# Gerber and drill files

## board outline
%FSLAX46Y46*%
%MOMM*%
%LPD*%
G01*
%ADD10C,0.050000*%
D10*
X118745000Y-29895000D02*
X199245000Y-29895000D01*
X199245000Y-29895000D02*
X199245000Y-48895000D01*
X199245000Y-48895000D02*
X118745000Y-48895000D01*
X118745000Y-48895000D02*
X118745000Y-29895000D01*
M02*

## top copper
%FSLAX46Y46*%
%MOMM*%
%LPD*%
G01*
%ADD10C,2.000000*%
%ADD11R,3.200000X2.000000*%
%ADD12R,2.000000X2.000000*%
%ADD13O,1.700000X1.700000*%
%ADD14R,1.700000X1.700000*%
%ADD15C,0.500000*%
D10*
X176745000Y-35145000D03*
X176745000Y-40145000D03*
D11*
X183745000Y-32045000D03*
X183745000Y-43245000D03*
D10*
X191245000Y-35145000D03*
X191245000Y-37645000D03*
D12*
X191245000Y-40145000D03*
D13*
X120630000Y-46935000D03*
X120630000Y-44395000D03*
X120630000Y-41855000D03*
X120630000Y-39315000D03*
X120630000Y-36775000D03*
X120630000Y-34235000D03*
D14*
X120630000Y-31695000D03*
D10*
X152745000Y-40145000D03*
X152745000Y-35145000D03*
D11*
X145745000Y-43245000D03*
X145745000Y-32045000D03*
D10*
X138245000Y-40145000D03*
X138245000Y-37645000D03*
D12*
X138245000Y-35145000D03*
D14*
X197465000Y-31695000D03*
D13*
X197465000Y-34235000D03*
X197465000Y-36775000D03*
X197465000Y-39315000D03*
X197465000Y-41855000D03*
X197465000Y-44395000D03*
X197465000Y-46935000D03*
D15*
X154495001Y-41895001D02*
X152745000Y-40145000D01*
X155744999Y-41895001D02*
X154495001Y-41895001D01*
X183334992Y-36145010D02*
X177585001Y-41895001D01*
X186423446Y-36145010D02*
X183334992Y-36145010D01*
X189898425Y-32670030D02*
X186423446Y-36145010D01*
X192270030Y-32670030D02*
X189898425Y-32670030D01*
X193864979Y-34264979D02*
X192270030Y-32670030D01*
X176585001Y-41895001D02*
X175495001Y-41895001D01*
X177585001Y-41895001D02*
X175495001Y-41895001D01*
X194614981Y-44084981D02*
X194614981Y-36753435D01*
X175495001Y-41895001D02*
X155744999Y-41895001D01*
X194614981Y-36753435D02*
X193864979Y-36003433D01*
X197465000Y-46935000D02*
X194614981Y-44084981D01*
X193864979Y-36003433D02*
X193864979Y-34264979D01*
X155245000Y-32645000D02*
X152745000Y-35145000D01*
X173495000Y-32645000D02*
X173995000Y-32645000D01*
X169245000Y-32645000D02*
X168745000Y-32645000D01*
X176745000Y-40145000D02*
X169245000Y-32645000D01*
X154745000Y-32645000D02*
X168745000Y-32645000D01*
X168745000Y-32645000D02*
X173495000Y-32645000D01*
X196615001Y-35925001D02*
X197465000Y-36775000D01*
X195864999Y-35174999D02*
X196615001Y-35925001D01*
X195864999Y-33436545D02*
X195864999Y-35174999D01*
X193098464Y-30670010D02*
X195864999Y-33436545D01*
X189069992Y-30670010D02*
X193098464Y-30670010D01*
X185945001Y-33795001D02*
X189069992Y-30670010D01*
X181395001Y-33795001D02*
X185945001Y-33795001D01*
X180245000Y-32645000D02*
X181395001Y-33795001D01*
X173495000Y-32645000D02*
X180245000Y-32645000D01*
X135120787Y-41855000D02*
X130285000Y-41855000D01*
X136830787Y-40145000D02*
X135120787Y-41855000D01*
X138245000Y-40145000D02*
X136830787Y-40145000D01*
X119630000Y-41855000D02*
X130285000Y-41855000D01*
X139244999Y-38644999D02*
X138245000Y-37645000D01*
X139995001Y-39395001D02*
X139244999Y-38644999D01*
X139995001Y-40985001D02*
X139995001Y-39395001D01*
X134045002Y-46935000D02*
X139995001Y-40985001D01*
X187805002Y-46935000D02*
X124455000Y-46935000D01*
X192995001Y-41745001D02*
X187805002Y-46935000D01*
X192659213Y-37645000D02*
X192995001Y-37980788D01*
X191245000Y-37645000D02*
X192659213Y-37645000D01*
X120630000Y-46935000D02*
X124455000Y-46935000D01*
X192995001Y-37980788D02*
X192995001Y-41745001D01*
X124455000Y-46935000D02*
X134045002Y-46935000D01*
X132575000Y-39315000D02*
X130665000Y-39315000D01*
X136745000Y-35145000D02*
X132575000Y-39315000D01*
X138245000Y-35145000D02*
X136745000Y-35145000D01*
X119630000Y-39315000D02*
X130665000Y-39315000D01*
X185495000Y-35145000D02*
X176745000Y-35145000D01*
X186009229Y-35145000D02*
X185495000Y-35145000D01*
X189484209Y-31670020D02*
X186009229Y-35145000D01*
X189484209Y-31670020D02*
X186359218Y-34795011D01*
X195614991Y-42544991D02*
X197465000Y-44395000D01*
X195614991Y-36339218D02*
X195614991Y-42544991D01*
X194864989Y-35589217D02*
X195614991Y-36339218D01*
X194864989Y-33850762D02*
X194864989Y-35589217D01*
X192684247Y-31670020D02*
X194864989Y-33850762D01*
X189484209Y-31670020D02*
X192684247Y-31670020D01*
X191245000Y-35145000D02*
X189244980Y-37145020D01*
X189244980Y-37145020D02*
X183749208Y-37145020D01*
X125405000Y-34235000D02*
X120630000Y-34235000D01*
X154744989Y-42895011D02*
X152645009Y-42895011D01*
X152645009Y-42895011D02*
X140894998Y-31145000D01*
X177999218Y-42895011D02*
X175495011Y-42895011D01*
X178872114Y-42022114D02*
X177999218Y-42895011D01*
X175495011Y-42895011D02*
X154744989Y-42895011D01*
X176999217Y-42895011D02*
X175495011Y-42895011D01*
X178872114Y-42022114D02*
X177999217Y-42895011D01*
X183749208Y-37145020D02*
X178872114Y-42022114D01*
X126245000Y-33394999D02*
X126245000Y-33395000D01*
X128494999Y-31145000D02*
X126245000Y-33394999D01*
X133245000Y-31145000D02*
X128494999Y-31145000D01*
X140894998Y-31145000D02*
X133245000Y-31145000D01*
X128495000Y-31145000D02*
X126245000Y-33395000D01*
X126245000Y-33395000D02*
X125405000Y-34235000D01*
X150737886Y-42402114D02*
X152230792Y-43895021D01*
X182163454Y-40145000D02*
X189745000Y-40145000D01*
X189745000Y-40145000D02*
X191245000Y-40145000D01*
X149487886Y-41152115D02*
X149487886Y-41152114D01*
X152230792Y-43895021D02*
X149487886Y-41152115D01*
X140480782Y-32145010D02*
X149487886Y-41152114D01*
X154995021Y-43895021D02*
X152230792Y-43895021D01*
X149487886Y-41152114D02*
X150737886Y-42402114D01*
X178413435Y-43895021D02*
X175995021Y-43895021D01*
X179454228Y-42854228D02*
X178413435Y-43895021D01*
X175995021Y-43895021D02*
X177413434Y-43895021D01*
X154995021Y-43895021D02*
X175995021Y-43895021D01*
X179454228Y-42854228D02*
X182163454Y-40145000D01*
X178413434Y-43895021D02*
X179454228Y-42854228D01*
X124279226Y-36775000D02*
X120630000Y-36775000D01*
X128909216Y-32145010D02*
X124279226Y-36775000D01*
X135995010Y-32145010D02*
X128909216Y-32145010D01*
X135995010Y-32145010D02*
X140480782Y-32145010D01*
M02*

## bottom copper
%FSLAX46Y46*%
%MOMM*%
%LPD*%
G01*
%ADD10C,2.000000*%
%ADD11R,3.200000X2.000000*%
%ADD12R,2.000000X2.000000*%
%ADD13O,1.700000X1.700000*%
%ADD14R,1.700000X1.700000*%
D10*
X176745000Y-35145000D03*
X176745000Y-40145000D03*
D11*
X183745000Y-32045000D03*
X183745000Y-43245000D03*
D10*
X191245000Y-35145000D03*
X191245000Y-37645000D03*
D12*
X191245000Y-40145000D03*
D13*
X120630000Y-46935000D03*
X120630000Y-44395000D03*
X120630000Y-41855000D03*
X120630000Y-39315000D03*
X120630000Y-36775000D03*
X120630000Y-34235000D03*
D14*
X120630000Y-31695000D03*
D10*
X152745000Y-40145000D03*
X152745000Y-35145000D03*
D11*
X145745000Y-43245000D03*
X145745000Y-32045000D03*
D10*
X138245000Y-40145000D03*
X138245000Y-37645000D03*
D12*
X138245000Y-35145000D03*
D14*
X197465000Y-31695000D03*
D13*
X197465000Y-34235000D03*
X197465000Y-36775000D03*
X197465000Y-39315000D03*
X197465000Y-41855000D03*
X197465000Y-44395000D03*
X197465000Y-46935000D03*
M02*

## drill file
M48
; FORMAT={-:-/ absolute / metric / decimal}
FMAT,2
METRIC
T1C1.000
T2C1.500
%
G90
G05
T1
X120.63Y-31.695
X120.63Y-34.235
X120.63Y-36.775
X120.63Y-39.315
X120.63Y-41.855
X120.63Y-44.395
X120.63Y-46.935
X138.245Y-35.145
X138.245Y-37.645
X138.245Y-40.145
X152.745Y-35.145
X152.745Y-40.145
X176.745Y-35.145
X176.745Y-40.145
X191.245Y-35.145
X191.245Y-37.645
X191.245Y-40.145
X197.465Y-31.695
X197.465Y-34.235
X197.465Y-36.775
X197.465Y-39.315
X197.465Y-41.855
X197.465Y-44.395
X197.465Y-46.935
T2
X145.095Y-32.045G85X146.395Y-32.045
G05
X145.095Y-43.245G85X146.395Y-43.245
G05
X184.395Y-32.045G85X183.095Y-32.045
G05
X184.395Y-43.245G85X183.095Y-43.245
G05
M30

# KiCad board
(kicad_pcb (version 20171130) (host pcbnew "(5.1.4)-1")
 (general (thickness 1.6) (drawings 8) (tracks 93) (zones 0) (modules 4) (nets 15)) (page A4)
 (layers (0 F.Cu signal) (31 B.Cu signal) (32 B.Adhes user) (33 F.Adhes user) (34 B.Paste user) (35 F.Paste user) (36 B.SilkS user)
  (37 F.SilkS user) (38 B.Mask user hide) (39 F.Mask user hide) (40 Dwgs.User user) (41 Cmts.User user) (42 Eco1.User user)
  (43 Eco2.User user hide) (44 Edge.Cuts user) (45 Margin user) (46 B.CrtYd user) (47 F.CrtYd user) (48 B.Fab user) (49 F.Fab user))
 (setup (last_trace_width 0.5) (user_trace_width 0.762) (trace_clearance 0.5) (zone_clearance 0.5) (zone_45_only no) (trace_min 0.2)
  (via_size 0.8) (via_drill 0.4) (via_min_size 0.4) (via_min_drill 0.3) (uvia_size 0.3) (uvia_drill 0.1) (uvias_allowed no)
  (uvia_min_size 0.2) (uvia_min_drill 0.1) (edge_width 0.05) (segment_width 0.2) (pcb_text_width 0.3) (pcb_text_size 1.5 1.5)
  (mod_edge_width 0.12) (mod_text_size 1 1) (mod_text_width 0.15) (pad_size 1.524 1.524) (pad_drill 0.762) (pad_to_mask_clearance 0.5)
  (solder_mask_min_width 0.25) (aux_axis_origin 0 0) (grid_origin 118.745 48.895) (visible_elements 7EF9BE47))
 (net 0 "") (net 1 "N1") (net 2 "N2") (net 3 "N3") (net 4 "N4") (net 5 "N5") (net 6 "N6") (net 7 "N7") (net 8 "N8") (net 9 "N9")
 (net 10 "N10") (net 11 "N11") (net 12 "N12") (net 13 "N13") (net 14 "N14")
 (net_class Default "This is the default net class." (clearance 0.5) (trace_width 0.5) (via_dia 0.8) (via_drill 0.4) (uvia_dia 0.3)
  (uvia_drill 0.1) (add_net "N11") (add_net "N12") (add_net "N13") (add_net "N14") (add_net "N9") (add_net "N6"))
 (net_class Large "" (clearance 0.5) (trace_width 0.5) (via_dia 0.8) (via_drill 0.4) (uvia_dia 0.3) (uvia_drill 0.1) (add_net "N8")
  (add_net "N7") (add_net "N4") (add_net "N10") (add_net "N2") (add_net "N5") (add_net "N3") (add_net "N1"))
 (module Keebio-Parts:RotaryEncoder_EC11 (layer F.Cu) (at 183.745 37.645 180)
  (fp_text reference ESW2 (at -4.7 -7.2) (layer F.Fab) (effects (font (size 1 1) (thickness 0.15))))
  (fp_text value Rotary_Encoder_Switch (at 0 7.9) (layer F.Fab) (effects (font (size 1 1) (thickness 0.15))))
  (pad S1 thru_hole circle (at 7 2.5 180) (size 2 2) (drill 1) (layers *.Cu *.Mask) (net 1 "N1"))
  (pad S2 thru_hole circle (at 7 -2.5 180) (size 2 2) (drill 1) (layers *.Cu *.Mask) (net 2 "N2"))
  (pad MP thru_hole rect (at 0 5.6 180) (size 3.2 2) (drill oval 2.8 1.5) (layers *.Cu *.Mask))
  (pad MP thru_hole rect (at 0 -5.6 180) (size 3.2 2) (drill oval 2.8 1.5) (layers *.Cu *.Mask))
  (pad B thru_hole circle (at -7.5 2.5 180) (size 2 2) (drill 1) (layers *.Cu *.Mask) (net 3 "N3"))
  (pad C thru_hole circle (at -7.5 0 180) (size 2 2) (drill 1) (layers *.Cu *.Mask) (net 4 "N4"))
  (pad A thru_hole rect (at -7.5 -2.5 180) (size 2 2) (drill 1) (layers *.Cu *.Mask) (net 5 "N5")))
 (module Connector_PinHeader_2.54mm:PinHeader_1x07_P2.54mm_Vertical (layer F.Cu) (at 120.63 31.695)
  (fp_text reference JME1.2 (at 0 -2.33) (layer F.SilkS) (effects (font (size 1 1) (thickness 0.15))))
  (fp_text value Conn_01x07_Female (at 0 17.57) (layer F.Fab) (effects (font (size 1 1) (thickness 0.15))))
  (pad 7 thru_hole oval (at 0 15.24) (size 1.7 1.7) (drill 1) (layers *.Cu *.Mask) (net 4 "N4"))
  (pad 6 thru_hole oval (at 0 12.7) (size 1.7 1.7) (drill 1) (layers *.Cu *.Mask) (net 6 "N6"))
  (pad 5 thru_hole oval (at 0 10.16) (size 1.7 1.7) (drill 1) (layers *.Cu *.Mask) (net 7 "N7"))
  (pad 4 thru_hole oval (at 0 7.62) (size 1.7 1.7) (drill 1) (layers *.Cu *.Mask) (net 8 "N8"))
  (pad 3 thru_hole oval (at 0 5.08) (size 1.7 1.7) (drill 1) (layers *.Cu *.Mask) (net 5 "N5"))
  (pad 2 thru_hole oval (at 0 2.54) (size 1.7 1.7) (drill 1) (layers *.Cu *.Mask) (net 3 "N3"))
  (pad 1 thru_hole rect (at 0 0) (size 1.7 1.7) (drill 1) (layers *.Cu *.Mask) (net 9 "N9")))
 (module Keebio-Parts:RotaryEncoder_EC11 (layer F.Cu) (at 145.745 37.645)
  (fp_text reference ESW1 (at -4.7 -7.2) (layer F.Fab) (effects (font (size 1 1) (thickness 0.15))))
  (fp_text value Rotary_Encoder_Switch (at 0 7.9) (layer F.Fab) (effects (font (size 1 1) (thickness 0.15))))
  (pad S1 thru_hole circle (at 7 2.5) (size 2 2) (drill 1) (layers *.Cu *.Mask) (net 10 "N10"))
  (pad S2 thru_hole circle (at 7 -2.5) (size 2 2) (drill 1) (layers *.Cu *.Mask) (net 2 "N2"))
  (pad MP thru_hole rect (at 0 5.6) (size 3.2 2) (drill oval 2.8 1.5) (layers *.Cu *.Mask))
  (pad MP thru_hole rect (at 0 -5.6) (size 3.2 2) (drill oval 2.8 1.5) (layers *.Cu *.Mask))
  (pad B thru_hole circle (at -7.5 2.5) (size 2 2) (drill 1) (layers *.Cu *.Mask) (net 7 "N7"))
  (pad C thru_hole circle (at -7.5 0) (size 2 2) (drill 1) (layers *.Cu *.Mask) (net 4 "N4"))
  (pad A thru_hole rect (at -7.5 -2.5) (size 2 2) (drill 1) (layers *.Cu *.Mask) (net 8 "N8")))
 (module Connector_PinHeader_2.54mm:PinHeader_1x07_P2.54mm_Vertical (layer F.Cu) (at 197.465 31.695)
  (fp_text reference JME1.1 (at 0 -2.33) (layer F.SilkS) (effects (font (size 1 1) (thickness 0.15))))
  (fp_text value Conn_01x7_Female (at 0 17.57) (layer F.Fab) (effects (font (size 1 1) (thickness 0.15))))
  (pad 1 thru_hole rect (at 0 0) (size 1.7 1.7) (drill 1) (layers *.Cu *.Mask) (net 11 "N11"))
  (pad 2 thru_hole oval (at 0 2.54) (size 1.7 1.7) (drill 1) (layers *.Cu *.Mask) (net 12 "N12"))
  (pad 3 thru_hole oval (at 0 5.08) (size 1.7 1.7) (drill 1) (layers *.Cu *.Mask) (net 2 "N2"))
  (pad 4 thru_hole oval (at 0 7.62) (size 1.7 1.7) (drill 1) (layers *.Cu *.Mask) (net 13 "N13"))
  (pad 5 thru_hole oval (at 0 10.16) (size 1.7 1.7) (drill 1) (layers *.Cu *.Mask) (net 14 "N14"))
  (pad 6 thru_hole oval (at 0 12.7) (size 1.7 1.7) (drill 1) (layers *.Cu *.Mask) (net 1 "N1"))
  (pad 7 thru_hole oval (at 0 15.24) (size 1.7 1.7) (drill 1) (layers *.Cu *.Mask) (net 10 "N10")))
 (gr_line (start 118.745 29.895) (end 199.245 29.895) (layer Edge.Cuts) (width 0.05))
 (gr_line (start 199.245 29.895) (end 199.245 48.895) (layer Edge.Cuts) (width 0.05))
 (gr_line (start 199.245 48.895) (end 118.745 48.895) (layer Edge.Cuts) (width 0.05))
 (gr_line (start 118.745 48.895) (end 118.745 29.895) (layer Edge.Cuts) (width 0.05))
 (segment (start 154.495001 41.895001) (end 152.745 40.145) (width 0.5) (layer F.Cu) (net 10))
 (segment (start 155.744999 41.895001) (end 154.495001 41.895001) (width 0.5) (layer F.Cu) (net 10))
 (segment (start 183.334992 36.14501) (end 177.585001 41.895001) (width 0.5) (layer F.Cu) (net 10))
 (segment (start 186.423446 36.14501) (end 183.334992 36.14501) (width 0.5) (layer F.Cu) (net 10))
 (segment (start 189.898425 32.67003) (end 186.423446 36.14501) (width 0.5) (layer F.Cu) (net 10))
 (segment (start 192.27003 32.67003) (end 189.898425 32.67003) (width 0.5) (layer F.Cu) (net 10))
 (segment (start 193.864979 34.264979) (end 192.27003 32.67003) (width 0.5) (layer F.Cu) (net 10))
 (segment (start 176.585001 41.895001) (end 175.495001 41.895001) (width 0.5) (layer F.Cu) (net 10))
 (segment (start 177.585001 41.895001) (end 175.495001 41.895001) (width 0.5) (layer F.Cu) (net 10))
 (segment (start 194.614981 44.084981) (end 194.614981 36.753435) (width 0.5) (layer F.Cu) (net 10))
 (segment (start 175.495001 41.895001) (end 155.744999 41.895001) (width 0.5) (layer F.Cu) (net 10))
 (segment (start 194.614981 36.753435) (end 193.864979 36.003433) (width 0.5) (layer F.Cu) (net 10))
 (segment (start 197.465 46.935) (end 194.614981 44.084981) (width 0.5) (layer F.Cu) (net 10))
 (segment (start 193.864979 36.003433) (end 193.864979 34.264979) (width 0.5) (layer F.Cu) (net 10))
 (segment (start 155.245 32.645) (end 152.745 35.145) (width 0.5) (layer F.Cu) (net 2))
 (segment (start 173.495 32.645) (end 173.995 32.645) (width 0.5) (layer F.Cu) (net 2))
 (segment (start 169.245 32.645) (end 168.745 32.645) (width 0.5) (layer F.Cu) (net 2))
 (segment (start 176.745 40.145) (end 169.245 32.645) (width 0.5) (layer F.Cu) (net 2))
 (segment (start 154.745 32.645) (end 168.745 32.645) (width 0.5) (layer F.Cu) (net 2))
 (segment (start 168.745 32.645) (end 173.495 32.645) (width 0.5) (layer F.Cu) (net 2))
 (segment (start 196.615001 35.925001) (end 197.465 36.775) (width 0.5) (layer F.Cu) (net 2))
 (segment (start 195.864999 35.174999) (end 196.615001 35.925001) (width 0.5) (layer F.Cu) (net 2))
 (segment (start 195.864999 33.436545) (end 195.864999 35.174999) (width 0.5) (layer F.Cu) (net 2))
 (segment (start 193.098464 30.67001) (end 195.864999 33.436545) (width 0.5) (layer F.Cu) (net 2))
 (segment (start 189.069992 30.67001) (end 193.098464 30.67001) (width 0.5) (layer F.Cu) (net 2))
 (segment (start 185.945001 33.795001) (end 189.069992 30.67001) (width 0.5) (layer F.Cu) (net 2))
 (segment (start 181.395001 33.795001) (end 185.945001 33.795001) (width 0.5) (layer F.Cu) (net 2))
 (segment (start 180.245 32.645) (end 181.395001 33.795001) (width 0.5) (layer F.Cu) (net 2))
 (segment (start 173.495 32.645) (end 180.245 32.645) (width 0.5) (layer F.Cu) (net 2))
 (segment (start 135.120787 41.855) (end 130.285 41.855) (width 0.5) (layer F.Cu) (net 7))
 (segment (start 136.830787 40.145) (end 135.120787 41.855) (width 0.5) (layer F.Cu) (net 7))
 (segment (start 138.245 40.145) (end 136.830787 40.145) (width 0.5) (layer F.Cu) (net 7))
 (segment (start 119.63 41.855) (end 130.285 41.855) (width 0.5) (layer F.Cu) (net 7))
 (segment (start 139.244999 38.644999) (end 138.245 37.645) (width 0.5) (layer F.Cu) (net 4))
 (segment (start 139.995001 39.395001) (end 139.244999 38.644999) (width 0.5) (layer F.Cu) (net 4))
 (segment (start 139.995001 40.985001) (end 139.995001 39.395001) (width 0.5) (layer F.Cu) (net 4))
 (segment (start 134.045002 46.935) (end 139.995001 40.985001) (width 0.5) (layer F.Cu) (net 4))
 (segment (start 187.805002 46.935) (end 124.455 46.935) (width 0.5) (layer F.Cu) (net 4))
 (segment (start 192.995001 41.745001) (end 187.805002 46.935) (width 0.5) (layer F.Cu) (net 4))
 (segment (start 192.659213 37.645) (end 192.995001 37.980788) (width 0.5) (layer F.Cu) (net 4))
 (segment (start 191.245 37.645) (end 192.659213 37.645) (width 0.5) (layer F.Cu) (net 4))
 (segment (start 120.63 46.935) (end 124.455 46.935) (width 0.5) (layer F.Cu) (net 4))
 (segment (start 192.995001 37.980788) (end 192.995001 41.745001) (width 0.5) (layer F.Cu) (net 4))
 (segment (start 124.455 46.935) (end 134.045002 46.935) (width 0.5) (layer F.Cu) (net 4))
 (segment (start 132.575 39.315) (end 130.665 39.315) (width 0.5) (layer F.Cu) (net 8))
 (segment (start 136.745 35.145) (end 132.575 39.315) (width 0.5) (layer F.Cu) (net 8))
 (segment (start 138.245 35.145) (end 136.745 35.145) (width 0.5) (layer F.Cu) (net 8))
 (segment (start 119.63 39.315) (end 130.665 39.315) (width 0.5) (layer F.Cu) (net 8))
 (segment (start 185.495 35.145) (end 176.745 35.145) (width 0.5) (layer F.Cu) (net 1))
 (segment (start 186.009229 35.145) (end 185.495 35.145) (width 0.5) (layer F.Cu) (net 1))
 (segment (start 189.484209 31.67002) (end 186.009229 35.145) (width 0.5) (layer F.Cu) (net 1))
 (segment (start 189.484209 31.67002) (end 186.359218 34.795011) (width 0.5) (layer F.Cu) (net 1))
 (segment (start 195.614991 42.544991) (end 197.465 44.395) (width 0.5) (layer F.Cu) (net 1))
 (segment (start 195.614991 36.339218) (end 195.614991 42.544991) (width 0.5) (layer F.Cu) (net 1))
 (segment (start 194.864989 35.589217) (end 195.614991 36.339218) (width 0.5) (layer F.Cu) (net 1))
 (segment (start 194.864989 33.850762) (end 194.864989 35.589217) (width 0.5) (layer F.Cu) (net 1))
 (segment (start 192.684247 31.67002) (end 194.864989 33.850762) (width 0.5) (layer F.Cu) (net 1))
 (segment (start 189.484209 31.67002) (end 192.684247 31.67002) (width 0.5) (layer F.Cu) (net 1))
 (segment (start 191.245 35.145) (end 189.24498 37.14502) (width 0.5) (layer F.Cu) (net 3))
 (segment (start 189.24498 37.14502) (end 183.749208 37.14502) (width 0.5) (layer F.Cu) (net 3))
 (segment (start 125.405 34.235) (end 120.63 34.235) (width 0.5) (layer F.Cu) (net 3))
 (segment (start 154.744989 42.895011) (end 152.645009 42.895011) (width 0.5) (layer F.Cu) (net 3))
 (segment (start 152.645009 42.895011) (end 140.894998 31.145) (width 0.5) (layer F.Cu) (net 3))
 (segment (start 177.999218 42.895011) (end 175.495011 42.895011) (width 0.5) (layer F.Cu) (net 3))
 (segment (start 178.872114 42.022114) (end 177.999218 42.895011) (width 0.5) (layer F.Cu) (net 3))
 (segment (start 175.495011 42.895011) (end 154.744989 42.895011) (width 0.5) (layer F.Cu) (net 3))
 (segment (start 176.999217 42.895011) (end 175.495011 42.895011) (width 0.5) (layer F.Cu) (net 3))
 (segment (start 178.872114 42.022114) (end 177.999217 42.895011) (width 0.5) (layer F.Cu) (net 3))
 (segment (start 183.749208 37.14502) (end 178.872114 42.022114) (width 0.5) (layer F.Cu) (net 3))
 (segment (start 126.245 33.394999) (end 126.245 33.395) (width 0.5) (layer F.Cu) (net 3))
 (segment (start 128.494999 31.145) (end 126.245 33.394999) (width 0.5) (layer F.Cu) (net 3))
 (segment (start 133.245 31.145) (end 128.494999 31.145) (width 0.5) (layer F.Cu) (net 3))
 (segment (start 140.894998 31.145) (end 133.245 31.145) (width 0.5) (layer F.Cu) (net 3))
 (segment (start 128.495 31.145) (end 126.245 33.395) (width 0.5) (layer F.Cu) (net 3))
 (segment (start 126.245 33.395) (end 125.405 34.235) (width 0.5) (layer F.Cu) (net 3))
 (segment (start 150.737886 42.402114) (end 152.230792 43.895021) (width 0.5) (layer F.Cu) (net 5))
 (segment (start 182.163454 40.145) (end 189.745 40.145) (width 0.5) (layer F.Cu) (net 5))
 (segment (start 189.745 40.145) (end 191.245 40.145) (width 0.5) (layer F.Cu) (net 5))
 (segment (start 149.487886 41.152115) (end 149.487886 41.152114) (width 0.5) (layer F.Cu) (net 5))
 (segment (start 152.230792 43.895021) (end 149.487886 41.152115) (width 0.5) (layer F.Cu) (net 5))
 (segment (start 140.480782 32.14501) (end 149.487886 41.152114) (width 0.5) (layer F.Cu) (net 5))
 (segment (start 154.995021 43.895021) (end 152.230792 43.895021) (width 0.5) (layer F.Cu) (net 5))
 (segment (start 149.487886 41.152114) (end 150.737886 42.402114) (width 0.5) (layer F.Cu) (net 5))
 (segment (start 178.413435 43.895021) (end 175.995021 43.895021) (width 0.5) (layer F.Cu) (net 5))
 (segment (start 179.454228 42.854228) (end 178.413435 43.895021) (width 0.5) (layer F.Cu) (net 5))
 (segment (start 175.995021 43.895021) (end 177.413434 43.895021) (width 0.5) (layer F.Cu) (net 5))
 (segment (start 154.995021 43.895021) (end 175.995021 43.895021) (width 0.5) (layer F.Cu) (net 5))
 (segment (start 179.454228 42.854228) (end 182.163454 40.145) (width 0.5) (layer F.Cu) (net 5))
 (segment (start 178.413434 43.895021) (end 179.454228 42.854228) (width 0.5) (layer F.Cu) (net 5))
 (segment (start 124.279226 36.775) (end 120.63 36.775) (width 0.5) (layer F.Cu) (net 5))
 (segment (start 128.909216 32.14501) (end 124.279226 36.775) (width 0.5) (layer F.Cu) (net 5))
 (segment (start 135.99501 32.14501) (end 128.909216 32.14501) (width 0.5) (layer F.Cu) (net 5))
 (segment (start 135.99501 32.14501) (end 140.480782 32.14501) (width 0.5) (layer F.Cu) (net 5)))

